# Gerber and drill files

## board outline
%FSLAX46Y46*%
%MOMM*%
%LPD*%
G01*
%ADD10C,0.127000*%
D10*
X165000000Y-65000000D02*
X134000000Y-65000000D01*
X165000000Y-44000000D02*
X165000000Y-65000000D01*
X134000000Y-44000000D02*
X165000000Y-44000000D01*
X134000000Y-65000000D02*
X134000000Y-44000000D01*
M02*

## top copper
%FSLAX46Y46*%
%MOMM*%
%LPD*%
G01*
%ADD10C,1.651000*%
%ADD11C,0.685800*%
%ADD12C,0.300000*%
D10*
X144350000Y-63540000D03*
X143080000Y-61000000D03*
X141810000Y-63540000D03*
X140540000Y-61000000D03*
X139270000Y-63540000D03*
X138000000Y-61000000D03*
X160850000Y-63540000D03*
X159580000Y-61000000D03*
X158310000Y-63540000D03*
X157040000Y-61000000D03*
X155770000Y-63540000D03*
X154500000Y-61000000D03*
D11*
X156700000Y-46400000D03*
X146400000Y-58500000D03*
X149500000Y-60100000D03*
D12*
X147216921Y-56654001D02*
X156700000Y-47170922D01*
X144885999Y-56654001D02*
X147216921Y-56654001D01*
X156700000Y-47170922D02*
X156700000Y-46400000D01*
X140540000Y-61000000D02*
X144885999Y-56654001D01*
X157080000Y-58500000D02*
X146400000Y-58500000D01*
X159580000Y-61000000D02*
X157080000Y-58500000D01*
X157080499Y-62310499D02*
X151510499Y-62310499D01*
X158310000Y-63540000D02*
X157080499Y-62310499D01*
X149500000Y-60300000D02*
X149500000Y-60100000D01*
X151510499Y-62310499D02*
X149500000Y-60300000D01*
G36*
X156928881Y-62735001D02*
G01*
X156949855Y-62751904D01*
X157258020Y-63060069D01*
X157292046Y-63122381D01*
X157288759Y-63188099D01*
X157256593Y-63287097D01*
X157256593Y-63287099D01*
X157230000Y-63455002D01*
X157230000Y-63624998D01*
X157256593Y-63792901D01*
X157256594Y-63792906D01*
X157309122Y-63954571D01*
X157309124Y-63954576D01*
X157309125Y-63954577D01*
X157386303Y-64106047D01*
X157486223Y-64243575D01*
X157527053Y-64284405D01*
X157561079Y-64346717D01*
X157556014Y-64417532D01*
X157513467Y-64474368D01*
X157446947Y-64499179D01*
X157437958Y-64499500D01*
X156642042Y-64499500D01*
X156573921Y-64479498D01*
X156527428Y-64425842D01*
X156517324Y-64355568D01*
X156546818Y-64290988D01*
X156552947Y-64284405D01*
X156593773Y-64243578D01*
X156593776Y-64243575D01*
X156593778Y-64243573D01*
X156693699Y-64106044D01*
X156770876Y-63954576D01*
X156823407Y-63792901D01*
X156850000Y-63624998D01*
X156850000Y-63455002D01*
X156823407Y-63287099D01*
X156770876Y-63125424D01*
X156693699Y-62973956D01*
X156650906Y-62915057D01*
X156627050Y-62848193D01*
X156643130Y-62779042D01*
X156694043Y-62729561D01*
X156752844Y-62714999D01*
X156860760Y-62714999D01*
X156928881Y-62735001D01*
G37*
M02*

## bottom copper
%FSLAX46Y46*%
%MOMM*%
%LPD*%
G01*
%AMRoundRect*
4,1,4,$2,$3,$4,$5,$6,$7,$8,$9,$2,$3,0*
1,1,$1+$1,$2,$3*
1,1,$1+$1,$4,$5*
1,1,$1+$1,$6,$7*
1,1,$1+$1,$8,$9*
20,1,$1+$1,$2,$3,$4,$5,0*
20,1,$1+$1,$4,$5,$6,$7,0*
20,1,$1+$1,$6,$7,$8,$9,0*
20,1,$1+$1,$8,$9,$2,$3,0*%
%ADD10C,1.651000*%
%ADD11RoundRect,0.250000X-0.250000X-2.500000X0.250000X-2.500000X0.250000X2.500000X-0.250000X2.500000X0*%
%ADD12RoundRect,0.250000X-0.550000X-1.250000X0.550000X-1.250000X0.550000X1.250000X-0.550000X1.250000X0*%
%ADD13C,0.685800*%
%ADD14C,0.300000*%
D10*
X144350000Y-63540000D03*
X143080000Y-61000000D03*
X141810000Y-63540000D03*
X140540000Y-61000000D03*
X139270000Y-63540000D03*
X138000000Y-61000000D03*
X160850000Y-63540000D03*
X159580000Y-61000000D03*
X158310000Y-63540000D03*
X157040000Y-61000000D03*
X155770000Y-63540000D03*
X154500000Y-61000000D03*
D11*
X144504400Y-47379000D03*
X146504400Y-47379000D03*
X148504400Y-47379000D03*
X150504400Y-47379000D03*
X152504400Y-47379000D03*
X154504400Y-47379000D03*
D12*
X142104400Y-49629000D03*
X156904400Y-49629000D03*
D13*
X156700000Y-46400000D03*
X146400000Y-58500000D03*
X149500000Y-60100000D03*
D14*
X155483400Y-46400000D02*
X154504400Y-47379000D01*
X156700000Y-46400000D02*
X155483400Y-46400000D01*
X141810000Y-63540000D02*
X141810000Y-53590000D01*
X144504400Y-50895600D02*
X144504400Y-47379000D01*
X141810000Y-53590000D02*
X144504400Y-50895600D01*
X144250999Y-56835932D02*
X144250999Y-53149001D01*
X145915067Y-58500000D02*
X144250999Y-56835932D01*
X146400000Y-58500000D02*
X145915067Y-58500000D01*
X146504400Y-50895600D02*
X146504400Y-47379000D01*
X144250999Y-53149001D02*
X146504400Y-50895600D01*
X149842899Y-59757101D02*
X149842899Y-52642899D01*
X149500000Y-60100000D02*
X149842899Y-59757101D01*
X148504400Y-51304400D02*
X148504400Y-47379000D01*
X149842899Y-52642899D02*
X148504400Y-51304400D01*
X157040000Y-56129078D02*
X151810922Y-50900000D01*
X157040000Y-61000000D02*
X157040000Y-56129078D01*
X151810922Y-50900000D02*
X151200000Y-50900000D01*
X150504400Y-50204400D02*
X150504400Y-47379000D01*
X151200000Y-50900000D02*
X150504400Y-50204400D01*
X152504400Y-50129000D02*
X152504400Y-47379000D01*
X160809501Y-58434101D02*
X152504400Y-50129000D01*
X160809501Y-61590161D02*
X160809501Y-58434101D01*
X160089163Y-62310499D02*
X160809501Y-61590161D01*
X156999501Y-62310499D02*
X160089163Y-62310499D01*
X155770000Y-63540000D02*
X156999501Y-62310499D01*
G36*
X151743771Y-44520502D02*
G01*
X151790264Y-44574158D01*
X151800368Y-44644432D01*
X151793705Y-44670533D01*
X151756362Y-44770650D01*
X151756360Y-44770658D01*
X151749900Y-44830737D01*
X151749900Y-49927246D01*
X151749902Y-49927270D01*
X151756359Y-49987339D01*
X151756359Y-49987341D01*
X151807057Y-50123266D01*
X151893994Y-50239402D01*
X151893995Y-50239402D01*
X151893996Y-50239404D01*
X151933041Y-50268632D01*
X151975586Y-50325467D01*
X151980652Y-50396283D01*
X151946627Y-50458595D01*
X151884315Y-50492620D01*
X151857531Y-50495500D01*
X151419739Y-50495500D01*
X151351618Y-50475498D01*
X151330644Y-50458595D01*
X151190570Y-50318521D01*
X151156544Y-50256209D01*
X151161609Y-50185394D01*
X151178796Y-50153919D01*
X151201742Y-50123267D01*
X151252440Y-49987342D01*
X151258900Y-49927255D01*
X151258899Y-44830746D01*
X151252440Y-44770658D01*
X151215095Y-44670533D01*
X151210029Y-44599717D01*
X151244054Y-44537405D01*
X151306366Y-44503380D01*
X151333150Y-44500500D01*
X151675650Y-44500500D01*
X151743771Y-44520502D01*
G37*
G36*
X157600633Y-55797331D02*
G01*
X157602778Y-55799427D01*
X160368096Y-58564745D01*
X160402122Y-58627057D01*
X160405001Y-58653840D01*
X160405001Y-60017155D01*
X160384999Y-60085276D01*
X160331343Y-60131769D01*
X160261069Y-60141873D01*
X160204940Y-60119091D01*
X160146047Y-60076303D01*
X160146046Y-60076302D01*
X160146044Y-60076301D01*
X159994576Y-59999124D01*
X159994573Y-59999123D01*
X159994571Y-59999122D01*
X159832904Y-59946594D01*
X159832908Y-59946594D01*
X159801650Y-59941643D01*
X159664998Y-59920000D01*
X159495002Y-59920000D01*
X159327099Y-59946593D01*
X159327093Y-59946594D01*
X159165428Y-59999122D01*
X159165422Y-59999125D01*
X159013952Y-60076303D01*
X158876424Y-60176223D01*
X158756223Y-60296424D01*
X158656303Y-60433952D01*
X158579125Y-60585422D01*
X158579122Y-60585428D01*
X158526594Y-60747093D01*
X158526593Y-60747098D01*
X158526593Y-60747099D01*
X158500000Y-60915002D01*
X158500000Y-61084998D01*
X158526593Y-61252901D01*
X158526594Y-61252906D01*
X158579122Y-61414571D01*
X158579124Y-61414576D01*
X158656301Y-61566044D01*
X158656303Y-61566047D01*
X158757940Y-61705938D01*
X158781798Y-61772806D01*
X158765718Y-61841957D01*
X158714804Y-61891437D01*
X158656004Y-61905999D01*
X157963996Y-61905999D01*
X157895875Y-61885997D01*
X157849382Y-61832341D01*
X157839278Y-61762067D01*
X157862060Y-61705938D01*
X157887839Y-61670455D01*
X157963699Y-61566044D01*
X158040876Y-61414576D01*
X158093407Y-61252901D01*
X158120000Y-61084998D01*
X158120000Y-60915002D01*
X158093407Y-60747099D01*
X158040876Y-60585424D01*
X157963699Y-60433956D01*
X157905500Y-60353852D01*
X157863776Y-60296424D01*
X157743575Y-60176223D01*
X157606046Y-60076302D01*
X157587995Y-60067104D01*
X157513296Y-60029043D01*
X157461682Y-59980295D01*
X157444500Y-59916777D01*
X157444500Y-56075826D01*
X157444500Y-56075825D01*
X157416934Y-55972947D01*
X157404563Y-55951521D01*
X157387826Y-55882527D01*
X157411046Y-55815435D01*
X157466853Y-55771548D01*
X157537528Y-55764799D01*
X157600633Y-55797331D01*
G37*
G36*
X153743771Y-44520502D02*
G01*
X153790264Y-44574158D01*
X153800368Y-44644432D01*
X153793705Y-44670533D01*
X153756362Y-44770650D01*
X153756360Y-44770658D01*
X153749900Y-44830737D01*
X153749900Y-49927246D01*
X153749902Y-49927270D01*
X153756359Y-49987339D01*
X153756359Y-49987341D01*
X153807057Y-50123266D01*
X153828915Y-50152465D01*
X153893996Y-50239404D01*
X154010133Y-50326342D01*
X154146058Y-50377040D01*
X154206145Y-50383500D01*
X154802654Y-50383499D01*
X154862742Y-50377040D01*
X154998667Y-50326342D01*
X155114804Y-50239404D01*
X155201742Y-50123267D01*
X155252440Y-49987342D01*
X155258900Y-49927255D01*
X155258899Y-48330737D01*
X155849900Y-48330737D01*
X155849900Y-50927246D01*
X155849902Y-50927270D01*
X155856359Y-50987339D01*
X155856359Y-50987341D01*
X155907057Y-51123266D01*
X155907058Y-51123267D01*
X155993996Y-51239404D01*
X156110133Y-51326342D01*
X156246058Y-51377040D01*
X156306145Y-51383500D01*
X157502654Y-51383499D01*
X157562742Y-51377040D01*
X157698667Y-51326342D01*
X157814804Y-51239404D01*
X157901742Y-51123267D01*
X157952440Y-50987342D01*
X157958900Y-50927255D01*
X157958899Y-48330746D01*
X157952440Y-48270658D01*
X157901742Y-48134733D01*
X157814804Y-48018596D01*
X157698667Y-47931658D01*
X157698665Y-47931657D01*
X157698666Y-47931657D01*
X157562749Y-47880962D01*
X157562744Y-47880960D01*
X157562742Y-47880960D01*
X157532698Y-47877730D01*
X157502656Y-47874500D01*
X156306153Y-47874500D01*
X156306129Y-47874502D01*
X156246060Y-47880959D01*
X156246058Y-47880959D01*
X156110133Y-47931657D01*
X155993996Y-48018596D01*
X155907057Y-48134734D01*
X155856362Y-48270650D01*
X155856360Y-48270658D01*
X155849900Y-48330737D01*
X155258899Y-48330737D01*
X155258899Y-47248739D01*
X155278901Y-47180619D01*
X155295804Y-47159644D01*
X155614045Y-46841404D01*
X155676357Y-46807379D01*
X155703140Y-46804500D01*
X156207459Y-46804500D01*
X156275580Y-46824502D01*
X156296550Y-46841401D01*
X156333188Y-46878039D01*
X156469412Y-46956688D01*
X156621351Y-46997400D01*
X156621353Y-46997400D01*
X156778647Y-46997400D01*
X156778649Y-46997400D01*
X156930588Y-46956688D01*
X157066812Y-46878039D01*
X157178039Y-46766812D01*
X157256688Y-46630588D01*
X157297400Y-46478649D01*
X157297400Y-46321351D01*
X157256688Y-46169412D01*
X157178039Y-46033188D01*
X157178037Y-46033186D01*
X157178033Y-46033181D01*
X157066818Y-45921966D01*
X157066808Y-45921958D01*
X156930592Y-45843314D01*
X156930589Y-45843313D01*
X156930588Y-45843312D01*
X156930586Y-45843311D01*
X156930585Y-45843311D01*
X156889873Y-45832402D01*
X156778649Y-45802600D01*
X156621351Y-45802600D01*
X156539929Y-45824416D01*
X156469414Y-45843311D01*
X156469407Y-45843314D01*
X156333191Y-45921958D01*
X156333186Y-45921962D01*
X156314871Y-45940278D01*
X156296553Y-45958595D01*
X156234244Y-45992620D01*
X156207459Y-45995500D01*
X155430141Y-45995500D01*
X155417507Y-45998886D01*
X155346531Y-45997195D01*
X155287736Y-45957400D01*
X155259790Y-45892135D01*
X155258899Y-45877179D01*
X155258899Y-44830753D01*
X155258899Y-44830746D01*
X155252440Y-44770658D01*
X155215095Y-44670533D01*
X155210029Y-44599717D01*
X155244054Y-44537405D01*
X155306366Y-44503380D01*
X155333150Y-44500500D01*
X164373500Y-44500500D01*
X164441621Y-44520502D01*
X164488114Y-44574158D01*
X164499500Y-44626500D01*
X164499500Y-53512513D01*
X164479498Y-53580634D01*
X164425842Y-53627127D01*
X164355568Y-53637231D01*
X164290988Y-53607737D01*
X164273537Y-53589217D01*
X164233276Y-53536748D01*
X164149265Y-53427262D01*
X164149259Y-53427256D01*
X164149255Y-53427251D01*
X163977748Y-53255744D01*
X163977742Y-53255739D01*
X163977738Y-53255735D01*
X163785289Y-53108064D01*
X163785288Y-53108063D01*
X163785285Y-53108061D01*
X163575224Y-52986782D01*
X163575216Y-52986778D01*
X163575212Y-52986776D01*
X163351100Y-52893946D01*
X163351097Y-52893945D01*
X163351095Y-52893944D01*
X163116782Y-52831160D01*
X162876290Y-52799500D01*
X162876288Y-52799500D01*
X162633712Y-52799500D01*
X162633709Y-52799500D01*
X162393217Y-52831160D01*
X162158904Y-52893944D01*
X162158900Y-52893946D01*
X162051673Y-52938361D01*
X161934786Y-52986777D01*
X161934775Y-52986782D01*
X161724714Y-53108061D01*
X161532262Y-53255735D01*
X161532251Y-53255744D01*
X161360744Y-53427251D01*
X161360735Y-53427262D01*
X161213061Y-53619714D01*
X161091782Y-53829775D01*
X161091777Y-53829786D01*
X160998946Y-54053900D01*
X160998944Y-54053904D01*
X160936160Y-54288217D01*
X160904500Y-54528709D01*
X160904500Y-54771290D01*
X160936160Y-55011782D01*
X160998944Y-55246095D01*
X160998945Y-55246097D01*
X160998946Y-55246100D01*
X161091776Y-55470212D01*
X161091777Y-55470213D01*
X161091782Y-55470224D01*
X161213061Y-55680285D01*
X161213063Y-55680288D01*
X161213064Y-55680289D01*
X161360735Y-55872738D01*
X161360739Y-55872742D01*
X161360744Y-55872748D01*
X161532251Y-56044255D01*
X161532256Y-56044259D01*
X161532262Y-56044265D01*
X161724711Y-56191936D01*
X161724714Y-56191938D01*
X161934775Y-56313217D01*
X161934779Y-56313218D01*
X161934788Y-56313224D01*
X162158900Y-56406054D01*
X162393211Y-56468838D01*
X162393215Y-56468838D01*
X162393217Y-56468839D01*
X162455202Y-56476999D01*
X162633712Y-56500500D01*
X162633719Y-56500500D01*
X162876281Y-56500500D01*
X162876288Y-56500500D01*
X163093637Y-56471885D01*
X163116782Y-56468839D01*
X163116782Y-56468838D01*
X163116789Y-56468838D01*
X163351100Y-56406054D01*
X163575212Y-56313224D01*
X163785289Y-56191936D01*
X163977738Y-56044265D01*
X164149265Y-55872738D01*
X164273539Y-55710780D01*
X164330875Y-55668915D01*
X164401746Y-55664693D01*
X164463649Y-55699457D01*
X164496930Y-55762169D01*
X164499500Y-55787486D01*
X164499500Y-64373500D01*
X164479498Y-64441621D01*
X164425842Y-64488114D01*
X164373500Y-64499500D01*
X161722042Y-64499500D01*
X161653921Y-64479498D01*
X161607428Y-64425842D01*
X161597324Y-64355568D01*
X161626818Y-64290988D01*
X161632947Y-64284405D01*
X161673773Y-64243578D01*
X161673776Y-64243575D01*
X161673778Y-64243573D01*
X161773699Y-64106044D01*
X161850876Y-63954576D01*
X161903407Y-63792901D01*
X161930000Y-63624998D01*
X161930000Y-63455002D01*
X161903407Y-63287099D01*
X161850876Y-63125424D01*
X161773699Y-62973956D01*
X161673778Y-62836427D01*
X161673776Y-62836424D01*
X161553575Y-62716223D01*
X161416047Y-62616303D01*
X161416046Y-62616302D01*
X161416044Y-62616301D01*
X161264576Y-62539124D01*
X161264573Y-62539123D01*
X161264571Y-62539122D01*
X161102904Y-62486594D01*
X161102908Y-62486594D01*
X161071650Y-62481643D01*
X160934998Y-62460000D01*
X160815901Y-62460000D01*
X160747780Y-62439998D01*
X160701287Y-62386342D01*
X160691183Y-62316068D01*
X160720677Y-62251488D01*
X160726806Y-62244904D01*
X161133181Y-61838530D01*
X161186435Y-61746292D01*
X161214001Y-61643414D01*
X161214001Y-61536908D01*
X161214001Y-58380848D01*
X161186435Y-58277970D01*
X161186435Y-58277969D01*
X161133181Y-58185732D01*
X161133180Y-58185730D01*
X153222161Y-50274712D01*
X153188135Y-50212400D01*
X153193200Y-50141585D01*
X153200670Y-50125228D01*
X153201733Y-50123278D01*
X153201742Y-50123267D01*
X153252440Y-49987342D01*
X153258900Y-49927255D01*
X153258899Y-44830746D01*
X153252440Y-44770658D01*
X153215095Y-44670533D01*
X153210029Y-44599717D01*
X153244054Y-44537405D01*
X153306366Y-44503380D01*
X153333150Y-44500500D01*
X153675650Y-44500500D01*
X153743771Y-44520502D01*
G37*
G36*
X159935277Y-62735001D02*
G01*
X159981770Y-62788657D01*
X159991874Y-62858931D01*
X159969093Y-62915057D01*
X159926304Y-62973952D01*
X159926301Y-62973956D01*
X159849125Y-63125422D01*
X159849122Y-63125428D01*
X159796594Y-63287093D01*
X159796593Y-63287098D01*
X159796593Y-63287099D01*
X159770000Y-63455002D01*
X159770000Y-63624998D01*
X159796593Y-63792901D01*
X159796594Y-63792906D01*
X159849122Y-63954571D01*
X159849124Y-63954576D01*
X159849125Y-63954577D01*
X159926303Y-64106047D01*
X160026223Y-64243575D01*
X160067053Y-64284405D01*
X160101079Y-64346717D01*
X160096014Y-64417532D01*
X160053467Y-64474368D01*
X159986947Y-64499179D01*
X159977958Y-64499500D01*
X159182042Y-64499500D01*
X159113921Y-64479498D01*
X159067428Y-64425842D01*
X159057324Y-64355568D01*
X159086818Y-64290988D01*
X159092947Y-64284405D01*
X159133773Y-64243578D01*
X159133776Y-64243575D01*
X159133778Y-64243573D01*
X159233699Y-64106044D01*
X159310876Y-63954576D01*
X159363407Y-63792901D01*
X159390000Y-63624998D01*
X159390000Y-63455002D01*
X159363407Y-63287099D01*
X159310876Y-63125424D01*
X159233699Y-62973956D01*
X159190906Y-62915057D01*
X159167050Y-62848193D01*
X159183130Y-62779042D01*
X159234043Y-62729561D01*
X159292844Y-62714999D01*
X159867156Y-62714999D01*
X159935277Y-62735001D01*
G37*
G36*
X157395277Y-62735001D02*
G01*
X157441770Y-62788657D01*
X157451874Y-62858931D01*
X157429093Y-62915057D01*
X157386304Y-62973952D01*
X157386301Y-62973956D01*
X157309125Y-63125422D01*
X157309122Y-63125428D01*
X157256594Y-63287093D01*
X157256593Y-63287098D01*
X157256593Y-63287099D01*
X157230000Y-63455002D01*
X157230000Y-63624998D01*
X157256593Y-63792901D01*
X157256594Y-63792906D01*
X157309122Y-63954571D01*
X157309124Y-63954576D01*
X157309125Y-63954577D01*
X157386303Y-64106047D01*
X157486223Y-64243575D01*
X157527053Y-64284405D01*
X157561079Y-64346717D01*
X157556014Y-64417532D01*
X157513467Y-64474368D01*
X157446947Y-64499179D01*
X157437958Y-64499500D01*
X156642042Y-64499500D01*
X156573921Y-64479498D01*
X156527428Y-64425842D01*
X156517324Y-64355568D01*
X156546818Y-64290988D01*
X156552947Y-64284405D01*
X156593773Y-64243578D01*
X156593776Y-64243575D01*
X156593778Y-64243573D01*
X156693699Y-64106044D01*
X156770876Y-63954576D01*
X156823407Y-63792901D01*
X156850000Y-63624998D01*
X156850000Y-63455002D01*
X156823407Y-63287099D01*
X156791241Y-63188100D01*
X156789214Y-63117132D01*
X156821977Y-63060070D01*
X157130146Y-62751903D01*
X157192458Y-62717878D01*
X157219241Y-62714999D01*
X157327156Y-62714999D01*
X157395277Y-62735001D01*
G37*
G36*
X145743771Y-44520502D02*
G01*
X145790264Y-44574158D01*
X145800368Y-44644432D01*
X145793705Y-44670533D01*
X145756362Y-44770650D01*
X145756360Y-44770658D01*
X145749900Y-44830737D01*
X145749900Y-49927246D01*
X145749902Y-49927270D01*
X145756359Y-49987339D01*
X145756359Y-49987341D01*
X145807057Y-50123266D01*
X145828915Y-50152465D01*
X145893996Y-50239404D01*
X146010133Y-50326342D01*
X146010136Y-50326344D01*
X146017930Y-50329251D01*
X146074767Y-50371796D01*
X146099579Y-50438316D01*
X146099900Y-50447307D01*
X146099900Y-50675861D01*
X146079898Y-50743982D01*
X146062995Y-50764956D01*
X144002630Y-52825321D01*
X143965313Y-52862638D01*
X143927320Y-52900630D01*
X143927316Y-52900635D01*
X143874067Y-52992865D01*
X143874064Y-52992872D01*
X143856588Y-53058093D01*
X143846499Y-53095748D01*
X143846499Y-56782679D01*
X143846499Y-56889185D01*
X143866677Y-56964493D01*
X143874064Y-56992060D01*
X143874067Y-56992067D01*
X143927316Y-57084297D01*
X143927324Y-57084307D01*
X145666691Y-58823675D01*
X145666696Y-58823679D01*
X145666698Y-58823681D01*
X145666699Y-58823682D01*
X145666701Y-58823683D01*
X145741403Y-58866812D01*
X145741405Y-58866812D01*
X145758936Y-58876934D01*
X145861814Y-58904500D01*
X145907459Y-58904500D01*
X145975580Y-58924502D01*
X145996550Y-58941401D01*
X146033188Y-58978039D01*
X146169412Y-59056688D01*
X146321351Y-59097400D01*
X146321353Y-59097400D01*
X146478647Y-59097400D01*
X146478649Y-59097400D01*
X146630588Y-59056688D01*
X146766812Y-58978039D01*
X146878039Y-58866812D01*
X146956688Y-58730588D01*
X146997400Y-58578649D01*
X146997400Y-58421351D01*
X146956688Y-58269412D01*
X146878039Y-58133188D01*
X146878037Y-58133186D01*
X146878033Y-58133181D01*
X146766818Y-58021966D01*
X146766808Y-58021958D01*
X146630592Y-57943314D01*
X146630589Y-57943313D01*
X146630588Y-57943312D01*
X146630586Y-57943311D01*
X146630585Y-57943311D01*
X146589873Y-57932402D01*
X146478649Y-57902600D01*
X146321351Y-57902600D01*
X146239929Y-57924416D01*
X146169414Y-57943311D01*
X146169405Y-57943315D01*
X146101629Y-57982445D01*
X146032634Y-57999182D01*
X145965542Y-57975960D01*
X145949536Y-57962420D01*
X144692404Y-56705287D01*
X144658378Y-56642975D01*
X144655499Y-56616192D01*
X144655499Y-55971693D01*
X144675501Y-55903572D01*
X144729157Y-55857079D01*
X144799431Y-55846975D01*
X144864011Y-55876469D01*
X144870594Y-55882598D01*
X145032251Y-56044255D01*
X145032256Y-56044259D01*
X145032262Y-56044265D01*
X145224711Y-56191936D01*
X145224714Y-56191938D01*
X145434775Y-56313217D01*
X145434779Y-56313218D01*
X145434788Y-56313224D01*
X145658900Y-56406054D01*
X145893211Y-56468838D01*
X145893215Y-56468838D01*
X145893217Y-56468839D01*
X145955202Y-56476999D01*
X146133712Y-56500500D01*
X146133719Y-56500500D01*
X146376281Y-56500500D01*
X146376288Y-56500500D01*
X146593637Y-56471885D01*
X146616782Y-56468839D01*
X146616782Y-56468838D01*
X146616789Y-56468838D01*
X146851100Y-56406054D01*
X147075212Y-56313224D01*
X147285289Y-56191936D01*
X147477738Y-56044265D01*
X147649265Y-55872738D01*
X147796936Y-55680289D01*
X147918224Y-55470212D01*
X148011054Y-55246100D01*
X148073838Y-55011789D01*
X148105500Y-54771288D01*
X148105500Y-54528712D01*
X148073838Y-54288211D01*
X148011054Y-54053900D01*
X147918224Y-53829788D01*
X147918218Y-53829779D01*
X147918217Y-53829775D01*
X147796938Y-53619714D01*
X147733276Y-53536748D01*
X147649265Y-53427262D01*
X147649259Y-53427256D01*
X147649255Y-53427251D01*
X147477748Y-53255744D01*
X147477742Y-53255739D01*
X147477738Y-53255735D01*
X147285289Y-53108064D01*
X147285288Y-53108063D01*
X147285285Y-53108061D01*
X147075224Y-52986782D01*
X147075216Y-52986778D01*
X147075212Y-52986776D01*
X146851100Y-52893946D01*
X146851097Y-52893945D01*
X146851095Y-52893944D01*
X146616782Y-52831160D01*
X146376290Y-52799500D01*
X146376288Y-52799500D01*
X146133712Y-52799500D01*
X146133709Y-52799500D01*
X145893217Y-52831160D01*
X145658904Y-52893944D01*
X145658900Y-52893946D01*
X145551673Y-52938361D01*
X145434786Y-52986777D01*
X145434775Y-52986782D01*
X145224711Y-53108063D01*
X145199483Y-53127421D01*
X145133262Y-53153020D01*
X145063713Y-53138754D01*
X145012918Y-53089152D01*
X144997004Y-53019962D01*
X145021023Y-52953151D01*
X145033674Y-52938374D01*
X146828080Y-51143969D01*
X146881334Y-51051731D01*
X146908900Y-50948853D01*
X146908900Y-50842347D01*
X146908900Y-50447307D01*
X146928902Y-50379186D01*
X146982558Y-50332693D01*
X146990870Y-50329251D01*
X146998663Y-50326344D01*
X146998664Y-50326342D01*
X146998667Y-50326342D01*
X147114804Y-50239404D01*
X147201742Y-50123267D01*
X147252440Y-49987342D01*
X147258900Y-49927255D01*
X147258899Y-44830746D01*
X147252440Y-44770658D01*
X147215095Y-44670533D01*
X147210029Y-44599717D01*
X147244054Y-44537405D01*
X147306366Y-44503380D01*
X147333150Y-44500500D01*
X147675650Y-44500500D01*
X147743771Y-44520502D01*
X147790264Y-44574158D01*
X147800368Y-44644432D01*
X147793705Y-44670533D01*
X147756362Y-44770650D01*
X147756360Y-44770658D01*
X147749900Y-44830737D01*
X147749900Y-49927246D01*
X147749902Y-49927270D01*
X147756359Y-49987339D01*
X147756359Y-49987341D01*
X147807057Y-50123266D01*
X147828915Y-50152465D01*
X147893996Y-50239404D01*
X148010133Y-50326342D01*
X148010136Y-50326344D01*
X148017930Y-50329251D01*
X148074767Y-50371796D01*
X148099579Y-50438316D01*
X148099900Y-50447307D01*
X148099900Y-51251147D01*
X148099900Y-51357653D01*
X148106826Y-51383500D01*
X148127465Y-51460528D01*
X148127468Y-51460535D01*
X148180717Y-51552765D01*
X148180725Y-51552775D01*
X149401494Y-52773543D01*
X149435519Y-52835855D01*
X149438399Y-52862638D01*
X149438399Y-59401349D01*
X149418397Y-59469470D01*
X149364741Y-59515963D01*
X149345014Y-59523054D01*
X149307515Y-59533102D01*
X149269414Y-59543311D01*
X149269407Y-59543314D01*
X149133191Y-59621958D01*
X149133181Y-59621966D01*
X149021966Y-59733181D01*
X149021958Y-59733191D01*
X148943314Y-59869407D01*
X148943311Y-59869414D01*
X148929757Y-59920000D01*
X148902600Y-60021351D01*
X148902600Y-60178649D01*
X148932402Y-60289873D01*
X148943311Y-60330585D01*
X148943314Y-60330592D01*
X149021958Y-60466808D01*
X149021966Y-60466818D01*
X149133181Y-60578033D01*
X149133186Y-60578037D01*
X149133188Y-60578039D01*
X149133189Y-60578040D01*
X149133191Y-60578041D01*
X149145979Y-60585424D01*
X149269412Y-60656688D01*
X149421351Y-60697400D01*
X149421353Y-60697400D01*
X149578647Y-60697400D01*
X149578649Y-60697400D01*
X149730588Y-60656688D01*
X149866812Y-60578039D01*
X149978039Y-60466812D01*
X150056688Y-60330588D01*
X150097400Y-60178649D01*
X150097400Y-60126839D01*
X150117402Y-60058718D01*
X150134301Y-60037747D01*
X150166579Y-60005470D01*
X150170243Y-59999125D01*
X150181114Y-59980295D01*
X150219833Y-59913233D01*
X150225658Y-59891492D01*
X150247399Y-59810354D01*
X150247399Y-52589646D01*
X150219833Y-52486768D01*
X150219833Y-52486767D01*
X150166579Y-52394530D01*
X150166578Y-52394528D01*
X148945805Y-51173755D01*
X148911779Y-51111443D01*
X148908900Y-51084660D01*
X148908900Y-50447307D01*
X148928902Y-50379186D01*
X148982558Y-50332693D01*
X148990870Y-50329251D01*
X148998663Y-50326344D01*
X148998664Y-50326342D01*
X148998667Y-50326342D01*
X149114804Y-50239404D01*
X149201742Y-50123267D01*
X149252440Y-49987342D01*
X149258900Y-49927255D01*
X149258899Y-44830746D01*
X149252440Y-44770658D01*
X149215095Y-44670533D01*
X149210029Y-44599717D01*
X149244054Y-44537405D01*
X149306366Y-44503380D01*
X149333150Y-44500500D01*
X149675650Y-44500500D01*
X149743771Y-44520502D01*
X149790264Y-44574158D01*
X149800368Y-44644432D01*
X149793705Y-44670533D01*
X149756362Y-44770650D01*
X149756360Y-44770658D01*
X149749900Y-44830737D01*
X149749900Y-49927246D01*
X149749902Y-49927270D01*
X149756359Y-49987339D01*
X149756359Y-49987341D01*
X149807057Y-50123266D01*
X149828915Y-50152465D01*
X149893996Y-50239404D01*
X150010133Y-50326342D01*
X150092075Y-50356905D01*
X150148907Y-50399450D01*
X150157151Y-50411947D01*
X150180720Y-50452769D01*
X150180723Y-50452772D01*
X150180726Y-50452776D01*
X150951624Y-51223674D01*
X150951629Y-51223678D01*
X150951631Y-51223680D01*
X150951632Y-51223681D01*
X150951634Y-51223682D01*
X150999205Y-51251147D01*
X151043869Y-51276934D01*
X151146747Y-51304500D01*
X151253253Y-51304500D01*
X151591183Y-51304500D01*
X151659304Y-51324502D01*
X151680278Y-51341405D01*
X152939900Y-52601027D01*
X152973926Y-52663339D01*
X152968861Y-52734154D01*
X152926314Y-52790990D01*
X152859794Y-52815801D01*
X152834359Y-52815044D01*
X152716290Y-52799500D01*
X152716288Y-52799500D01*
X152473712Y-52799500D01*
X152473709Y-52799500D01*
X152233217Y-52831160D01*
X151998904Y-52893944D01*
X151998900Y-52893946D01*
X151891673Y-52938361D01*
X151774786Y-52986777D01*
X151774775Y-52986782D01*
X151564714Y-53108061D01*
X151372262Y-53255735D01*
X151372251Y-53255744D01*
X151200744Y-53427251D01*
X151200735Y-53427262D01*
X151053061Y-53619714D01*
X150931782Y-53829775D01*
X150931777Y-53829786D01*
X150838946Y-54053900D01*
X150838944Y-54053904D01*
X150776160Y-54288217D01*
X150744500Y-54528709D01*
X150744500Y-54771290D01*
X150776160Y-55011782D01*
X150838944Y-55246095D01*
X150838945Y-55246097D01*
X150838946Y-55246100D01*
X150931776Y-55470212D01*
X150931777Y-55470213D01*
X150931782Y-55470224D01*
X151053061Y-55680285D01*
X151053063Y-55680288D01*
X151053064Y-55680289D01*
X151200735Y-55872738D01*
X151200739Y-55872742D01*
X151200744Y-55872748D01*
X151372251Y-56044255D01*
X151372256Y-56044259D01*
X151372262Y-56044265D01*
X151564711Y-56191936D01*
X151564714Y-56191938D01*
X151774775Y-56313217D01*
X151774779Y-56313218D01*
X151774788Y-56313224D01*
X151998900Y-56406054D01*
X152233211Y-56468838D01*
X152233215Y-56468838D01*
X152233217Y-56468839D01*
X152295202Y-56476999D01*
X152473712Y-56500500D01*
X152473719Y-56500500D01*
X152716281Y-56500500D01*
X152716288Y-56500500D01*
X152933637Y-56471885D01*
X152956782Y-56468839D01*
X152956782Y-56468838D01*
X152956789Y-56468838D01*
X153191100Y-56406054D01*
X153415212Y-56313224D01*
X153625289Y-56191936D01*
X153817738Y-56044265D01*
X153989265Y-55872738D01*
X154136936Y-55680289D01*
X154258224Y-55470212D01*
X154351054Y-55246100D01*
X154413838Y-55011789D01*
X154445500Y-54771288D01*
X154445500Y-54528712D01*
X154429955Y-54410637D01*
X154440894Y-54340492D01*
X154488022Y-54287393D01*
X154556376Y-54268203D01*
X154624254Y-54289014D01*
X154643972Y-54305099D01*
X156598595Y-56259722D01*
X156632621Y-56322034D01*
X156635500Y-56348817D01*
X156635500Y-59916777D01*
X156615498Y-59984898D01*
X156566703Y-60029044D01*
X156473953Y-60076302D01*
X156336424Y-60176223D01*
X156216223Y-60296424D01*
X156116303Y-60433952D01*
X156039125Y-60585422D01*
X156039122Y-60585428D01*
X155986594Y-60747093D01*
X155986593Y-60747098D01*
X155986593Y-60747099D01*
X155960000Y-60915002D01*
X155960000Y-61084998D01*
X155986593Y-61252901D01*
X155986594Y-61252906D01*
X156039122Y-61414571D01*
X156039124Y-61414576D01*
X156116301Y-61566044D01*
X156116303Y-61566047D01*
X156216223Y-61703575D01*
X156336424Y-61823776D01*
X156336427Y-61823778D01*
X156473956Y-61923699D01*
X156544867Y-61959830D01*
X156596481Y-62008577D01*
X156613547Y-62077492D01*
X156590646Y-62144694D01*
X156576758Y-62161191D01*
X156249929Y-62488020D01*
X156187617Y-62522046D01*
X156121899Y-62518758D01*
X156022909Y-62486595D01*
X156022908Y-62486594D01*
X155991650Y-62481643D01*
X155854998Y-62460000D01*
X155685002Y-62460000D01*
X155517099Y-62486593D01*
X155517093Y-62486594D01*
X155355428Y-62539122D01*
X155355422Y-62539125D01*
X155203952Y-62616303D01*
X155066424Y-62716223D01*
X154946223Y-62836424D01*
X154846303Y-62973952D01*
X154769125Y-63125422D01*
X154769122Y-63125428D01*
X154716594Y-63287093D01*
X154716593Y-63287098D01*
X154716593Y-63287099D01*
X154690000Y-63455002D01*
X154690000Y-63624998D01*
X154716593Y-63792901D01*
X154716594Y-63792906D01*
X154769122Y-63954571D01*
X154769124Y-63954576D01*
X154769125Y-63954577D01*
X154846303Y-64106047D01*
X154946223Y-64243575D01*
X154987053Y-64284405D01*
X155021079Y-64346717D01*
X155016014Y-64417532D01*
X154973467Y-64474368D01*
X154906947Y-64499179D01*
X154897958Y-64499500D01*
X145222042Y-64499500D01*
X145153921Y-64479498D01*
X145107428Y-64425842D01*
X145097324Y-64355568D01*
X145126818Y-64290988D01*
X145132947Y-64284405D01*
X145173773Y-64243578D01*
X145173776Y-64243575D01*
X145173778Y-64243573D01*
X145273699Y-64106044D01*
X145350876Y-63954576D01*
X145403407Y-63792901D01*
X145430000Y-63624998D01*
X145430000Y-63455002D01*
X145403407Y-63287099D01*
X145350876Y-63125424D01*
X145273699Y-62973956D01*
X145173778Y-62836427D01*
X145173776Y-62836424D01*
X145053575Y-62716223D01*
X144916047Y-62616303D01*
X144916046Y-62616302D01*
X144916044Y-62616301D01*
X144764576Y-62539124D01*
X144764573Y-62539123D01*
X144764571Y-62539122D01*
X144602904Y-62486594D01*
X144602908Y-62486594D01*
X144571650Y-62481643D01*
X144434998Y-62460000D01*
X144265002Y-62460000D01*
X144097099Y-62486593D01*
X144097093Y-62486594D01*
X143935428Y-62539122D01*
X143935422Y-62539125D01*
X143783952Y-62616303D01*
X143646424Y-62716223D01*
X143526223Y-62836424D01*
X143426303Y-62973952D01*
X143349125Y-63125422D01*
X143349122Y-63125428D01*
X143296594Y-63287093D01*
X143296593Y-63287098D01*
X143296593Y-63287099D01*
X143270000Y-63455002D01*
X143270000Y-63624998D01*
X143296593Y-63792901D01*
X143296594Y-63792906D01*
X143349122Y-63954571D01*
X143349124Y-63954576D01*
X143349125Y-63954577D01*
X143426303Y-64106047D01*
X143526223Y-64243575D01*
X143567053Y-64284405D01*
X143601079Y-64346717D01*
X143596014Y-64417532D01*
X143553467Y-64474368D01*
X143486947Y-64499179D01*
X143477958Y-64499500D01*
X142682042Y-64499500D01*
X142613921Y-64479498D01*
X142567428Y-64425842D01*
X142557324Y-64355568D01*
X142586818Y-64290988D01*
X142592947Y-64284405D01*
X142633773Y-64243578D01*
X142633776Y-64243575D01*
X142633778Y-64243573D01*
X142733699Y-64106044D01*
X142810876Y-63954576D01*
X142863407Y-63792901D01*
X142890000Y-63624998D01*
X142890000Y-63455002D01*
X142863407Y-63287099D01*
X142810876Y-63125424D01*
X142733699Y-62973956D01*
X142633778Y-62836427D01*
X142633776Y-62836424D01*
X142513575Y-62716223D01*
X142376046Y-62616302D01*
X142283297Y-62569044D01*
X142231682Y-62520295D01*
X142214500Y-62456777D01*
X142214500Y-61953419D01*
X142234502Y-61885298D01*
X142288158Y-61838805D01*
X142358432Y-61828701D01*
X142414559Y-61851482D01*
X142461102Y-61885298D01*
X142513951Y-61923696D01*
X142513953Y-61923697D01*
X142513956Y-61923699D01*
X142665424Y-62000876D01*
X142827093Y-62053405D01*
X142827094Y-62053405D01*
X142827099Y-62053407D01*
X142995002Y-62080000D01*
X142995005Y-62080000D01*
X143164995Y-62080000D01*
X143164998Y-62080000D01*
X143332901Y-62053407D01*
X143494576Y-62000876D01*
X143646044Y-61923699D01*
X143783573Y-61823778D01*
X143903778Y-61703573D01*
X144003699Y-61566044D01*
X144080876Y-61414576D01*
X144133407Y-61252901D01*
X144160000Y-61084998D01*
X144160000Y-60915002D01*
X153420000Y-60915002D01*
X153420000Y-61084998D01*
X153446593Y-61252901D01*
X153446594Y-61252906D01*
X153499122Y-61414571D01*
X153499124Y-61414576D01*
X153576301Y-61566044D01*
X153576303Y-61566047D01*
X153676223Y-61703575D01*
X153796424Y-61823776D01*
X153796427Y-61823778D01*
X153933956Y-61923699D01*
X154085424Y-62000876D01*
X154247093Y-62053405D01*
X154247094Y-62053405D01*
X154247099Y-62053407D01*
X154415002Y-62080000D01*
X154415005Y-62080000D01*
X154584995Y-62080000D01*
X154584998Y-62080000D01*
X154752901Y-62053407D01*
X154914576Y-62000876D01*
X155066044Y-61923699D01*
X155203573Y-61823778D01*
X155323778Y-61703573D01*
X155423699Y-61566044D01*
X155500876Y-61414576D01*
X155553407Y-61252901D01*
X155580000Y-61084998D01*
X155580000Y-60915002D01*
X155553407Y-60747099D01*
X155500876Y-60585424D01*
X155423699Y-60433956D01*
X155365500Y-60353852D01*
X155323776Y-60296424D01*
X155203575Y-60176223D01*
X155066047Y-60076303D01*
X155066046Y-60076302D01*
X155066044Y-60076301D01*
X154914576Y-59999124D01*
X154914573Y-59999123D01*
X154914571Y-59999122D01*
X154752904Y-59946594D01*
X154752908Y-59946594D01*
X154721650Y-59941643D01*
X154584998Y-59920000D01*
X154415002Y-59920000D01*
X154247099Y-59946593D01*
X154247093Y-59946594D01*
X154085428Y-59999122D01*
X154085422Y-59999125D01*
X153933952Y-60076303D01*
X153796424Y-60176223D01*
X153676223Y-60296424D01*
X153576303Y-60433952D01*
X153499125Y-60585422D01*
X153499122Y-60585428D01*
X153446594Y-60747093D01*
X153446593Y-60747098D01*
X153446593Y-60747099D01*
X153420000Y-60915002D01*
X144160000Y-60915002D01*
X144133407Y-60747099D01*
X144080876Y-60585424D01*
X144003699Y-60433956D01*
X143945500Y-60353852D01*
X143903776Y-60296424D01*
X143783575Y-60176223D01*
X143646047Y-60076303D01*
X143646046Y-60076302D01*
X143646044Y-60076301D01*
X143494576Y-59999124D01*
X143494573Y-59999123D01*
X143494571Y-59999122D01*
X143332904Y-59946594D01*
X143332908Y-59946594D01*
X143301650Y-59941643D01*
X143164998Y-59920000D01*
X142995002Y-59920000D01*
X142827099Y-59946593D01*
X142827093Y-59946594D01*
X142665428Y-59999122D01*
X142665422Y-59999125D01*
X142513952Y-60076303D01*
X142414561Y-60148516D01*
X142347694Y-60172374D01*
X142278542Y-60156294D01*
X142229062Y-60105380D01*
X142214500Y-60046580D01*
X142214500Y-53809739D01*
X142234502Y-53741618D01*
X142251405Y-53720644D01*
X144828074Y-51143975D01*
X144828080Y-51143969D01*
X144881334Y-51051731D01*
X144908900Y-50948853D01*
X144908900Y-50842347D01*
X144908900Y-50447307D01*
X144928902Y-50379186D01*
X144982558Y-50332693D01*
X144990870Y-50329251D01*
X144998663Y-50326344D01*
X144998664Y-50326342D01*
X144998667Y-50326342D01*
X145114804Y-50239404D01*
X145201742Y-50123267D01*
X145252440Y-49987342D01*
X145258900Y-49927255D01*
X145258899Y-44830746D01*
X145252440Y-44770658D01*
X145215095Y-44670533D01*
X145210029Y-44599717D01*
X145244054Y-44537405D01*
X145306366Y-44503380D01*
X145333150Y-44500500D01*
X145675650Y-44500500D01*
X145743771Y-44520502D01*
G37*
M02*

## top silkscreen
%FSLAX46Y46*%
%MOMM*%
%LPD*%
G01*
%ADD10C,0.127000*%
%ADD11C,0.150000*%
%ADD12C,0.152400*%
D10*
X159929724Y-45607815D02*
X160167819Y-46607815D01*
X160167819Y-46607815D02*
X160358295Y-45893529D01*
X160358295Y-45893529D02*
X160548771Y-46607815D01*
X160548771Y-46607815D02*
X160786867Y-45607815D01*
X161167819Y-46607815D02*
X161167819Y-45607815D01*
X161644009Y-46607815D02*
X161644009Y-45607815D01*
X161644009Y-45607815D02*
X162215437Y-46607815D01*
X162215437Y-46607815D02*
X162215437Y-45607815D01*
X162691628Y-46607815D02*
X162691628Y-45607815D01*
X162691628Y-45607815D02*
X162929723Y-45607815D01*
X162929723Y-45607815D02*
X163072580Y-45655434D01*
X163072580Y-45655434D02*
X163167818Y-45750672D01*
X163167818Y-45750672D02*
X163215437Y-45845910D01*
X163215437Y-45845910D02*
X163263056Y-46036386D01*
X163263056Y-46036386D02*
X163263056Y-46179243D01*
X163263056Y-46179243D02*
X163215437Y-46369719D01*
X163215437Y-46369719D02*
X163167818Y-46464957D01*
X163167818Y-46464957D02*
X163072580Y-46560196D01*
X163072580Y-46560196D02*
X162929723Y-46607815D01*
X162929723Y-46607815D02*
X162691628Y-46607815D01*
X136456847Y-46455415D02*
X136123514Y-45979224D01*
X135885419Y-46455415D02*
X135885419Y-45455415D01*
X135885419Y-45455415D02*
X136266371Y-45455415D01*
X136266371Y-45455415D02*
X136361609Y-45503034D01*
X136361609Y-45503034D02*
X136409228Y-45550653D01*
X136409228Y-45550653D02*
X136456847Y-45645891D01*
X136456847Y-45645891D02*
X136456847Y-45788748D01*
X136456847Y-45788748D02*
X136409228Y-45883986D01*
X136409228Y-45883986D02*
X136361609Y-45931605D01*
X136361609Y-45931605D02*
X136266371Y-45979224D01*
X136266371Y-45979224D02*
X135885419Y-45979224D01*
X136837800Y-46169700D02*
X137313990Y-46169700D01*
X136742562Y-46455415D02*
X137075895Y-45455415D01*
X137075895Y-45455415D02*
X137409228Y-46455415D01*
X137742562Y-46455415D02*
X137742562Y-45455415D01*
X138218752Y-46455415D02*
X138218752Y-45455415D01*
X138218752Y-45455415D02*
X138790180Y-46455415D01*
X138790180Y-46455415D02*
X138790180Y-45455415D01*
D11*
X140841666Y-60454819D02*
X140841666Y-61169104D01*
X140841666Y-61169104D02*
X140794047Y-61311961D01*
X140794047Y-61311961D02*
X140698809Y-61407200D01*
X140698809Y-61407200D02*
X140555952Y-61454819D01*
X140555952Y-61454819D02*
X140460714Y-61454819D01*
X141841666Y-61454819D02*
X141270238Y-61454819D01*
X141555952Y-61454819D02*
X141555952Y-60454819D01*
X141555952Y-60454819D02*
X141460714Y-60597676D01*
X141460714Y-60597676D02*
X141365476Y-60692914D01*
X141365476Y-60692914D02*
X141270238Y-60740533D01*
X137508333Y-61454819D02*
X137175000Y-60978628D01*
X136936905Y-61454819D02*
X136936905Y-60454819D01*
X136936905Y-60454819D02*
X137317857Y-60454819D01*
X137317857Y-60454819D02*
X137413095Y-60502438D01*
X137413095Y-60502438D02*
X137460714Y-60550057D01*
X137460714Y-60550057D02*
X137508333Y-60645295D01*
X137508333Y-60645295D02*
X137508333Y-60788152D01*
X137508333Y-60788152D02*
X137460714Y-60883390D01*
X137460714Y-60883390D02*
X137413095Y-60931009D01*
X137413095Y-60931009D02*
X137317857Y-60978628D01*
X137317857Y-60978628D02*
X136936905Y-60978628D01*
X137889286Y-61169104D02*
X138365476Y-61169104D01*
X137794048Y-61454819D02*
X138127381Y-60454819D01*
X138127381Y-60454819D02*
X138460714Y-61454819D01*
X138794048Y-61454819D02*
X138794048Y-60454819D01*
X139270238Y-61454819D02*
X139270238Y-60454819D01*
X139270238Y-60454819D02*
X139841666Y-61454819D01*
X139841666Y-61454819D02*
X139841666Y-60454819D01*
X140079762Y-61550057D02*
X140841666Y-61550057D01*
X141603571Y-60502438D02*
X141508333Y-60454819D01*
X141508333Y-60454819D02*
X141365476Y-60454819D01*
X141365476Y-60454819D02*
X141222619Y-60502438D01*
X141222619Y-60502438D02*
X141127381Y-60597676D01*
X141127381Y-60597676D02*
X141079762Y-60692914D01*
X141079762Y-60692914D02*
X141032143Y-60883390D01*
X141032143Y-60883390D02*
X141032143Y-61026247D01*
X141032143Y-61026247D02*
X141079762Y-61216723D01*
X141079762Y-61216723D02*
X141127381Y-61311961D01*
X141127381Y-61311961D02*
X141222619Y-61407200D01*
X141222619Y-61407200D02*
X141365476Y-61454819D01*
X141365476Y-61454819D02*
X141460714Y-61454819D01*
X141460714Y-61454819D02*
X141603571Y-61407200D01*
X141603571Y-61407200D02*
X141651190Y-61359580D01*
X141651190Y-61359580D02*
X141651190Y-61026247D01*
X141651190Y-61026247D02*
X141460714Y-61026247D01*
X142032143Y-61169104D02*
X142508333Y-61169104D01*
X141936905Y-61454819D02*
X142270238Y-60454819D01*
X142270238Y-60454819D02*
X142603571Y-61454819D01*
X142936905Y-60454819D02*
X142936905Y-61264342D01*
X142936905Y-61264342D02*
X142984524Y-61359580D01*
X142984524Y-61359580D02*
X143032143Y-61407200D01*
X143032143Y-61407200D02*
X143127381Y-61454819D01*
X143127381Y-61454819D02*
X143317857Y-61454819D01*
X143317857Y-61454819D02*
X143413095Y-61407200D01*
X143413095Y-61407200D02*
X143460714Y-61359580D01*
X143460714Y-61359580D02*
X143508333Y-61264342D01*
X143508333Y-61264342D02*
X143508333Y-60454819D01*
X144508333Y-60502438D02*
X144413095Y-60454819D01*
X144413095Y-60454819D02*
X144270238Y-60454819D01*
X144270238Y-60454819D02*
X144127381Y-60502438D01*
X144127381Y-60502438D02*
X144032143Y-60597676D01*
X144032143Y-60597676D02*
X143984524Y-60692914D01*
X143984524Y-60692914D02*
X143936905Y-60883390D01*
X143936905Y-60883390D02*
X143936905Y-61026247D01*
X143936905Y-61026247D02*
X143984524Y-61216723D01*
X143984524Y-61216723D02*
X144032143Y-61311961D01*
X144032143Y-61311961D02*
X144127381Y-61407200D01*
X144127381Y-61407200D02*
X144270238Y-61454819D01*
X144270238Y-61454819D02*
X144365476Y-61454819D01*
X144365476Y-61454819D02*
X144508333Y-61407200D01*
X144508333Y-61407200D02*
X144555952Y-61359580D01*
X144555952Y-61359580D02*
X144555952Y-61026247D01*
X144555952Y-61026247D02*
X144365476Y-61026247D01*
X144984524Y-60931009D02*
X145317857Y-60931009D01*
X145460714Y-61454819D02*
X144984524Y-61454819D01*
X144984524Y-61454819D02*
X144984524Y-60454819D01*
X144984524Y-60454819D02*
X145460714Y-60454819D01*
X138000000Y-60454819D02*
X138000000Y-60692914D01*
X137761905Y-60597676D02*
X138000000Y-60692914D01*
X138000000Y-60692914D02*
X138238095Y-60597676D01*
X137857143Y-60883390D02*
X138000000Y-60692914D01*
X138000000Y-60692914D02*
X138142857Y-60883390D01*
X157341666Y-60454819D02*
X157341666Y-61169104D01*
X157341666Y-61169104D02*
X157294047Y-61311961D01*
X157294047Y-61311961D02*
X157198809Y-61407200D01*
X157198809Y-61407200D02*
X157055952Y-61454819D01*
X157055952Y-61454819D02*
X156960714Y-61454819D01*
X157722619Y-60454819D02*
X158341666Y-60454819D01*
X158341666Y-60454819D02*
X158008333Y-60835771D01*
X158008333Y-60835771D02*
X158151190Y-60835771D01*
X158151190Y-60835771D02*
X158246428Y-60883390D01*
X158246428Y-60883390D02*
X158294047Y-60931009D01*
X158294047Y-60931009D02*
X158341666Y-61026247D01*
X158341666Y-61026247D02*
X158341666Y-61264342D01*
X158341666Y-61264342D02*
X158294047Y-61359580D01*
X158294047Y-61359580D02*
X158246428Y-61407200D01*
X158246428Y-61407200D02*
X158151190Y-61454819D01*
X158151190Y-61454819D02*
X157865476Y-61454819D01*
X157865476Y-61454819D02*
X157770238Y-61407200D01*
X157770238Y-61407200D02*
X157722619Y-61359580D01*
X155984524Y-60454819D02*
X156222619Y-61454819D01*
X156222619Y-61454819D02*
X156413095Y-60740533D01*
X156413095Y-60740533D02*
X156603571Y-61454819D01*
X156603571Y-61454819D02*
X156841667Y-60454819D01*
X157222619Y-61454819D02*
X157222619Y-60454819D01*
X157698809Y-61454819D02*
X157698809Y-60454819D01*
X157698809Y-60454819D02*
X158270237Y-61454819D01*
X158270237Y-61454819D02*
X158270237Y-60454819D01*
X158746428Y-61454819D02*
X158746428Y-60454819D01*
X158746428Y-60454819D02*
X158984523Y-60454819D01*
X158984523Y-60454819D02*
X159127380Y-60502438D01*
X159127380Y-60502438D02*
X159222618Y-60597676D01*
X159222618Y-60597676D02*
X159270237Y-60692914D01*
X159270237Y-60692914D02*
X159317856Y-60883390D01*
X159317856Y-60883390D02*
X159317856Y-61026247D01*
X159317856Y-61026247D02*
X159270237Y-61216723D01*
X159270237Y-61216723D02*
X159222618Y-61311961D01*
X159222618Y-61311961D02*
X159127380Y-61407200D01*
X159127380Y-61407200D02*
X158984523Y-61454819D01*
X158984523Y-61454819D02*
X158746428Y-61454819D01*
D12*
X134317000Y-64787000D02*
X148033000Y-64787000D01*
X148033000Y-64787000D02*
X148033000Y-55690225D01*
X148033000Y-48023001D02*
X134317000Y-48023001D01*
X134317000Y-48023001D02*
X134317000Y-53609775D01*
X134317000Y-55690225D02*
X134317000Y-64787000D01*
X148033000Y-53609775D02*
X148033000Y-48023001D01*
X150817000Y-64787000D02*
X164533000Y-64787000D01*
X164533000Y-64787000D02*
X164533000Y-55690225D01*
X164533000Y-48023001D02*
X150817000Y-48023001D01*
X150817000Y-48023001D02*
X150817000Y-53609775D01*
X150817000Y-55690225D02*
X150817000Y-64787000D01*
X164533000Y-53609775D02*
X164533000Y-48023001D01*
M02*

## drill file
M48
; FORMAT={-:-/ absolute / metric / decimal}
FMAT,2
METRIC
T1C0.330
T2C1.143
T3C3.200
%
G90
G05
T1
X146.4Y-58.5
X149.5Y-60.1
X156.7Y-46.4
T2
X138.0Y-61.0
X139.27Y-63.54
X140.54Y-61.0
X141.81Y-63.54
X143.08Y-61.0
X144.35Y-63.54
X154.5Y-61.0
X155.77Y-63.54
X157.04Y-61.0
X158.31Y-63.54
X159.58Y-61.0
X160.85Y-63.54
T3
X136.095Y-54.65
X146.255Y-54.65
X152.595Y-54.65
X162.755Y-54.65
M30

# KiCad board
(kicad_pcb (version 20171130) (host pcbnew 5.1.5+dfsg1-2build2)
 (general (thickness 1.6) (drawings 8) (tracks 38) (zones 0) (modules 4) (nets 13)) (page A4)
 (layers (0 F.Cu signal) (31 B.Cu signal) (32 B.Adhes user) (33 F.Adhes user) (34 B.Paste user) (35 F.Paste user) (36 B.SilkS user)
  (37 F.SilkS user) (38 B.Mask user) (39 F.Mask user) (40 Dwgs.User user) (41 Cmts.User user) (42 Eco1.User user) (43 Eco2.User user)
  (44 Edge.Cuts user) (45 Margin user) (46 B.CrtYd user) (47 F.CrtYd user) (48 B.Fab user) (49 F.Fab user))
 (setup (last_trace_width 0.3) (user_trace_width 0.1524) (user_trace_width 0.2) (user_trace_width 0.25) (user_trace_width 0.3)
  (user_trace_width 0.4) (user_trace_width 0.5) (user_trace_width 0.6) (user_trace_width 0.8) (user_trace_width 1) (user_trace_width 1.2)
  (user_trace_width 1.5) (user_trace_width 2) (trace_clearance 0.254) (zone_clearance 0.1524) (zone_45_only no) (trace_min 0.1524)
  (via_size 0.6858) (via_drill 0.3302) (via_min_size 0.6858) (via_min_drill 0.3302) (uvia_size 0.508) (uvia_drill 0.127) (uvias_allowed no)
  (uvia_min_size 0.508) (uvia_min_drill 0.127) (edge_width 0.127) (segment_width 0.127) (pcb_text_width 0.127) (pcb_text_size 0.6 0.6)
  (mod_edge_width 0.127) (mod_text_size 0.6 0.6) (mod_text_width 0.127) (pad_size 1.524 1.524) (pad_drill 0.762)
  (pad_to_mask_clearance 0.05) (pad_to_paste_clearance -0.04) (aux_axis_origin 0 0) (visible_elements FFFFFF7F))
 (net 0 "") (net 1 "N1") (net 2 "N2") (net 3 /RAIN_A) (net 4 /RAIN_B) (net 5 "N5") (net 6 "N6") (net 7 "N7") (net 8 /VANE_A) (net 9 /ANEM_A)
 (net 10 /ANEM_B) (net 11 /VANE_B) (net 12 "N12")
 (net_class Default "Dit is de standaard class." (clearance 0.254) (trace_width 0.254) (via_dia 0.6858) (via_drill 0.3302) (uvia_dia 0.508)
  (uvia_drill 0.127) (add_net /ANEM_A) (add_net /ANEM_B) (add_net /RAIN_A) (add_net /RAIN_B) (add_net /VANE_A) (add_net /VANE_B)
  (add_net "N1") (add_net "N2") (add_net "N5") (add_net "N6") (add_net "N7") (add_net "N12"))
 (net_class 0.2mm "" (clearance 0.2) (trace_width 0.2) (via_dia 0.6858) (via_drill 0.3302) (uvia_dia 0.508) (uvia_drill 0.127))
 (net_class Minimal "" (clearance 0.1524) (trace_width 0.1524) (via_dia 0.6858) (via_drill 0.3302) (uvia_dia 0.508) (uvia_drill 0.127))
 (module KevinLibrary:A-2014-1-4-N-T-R (layer F.Cu) (at 138 61)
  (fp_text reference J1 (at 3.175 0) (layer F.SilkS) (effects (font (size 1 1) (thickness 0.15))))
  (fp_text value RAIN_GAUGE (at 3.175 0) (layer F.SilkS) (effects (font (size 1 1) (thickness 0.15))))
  (fp_line (start -3.683 3.787) (end 10.033 3.787) (layer F.SilkS) (width 0.1524))
  (fp_line (start 10.033 3.787) (end 10.033 -5.309775) (layer F.SilkS) (width 0.1524))
  (fp_line (start 10.033 -12.976999) (end -3.683 -12.976999) (layer F.SilkS) (width 0.1524))
  (fp_line (start -3.683 -12.976999) (end -3.683 -7.390225) (layer F.SilkS) (width 0.1524))
  (fp_line (start -3.683 -5.309775) (end -3.683 3.787) (layer F.SilkS) (width 0.1524))
  (fp_line (start 10.033 -7.390225) (end 10.033 -12.976999) (layer F.SilkS) (width 0.1524))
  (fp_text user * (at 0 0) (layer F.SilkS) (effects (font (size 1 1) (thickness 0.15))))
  (pad 1 thru_hole circle (at 6.35 2.54) (size 1.651 1.651) (drill 1.143) (layers *.Cu *.Mask) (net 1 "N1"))
  (pad 2 thru_hole circle (at 5.08 0) (size 1.651 1.651) (drill 1.143) (layers *.Cu *.Mask) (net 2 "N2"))
  (pad 3 thru_hole circle (at 3.81 2.54) (size 1.651 1.651) (drill 1.143) (layers *.Cu *.Mask) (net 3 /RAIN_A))
  (pad 4 thru_hole circle (at 2.54 0) (size 1.651 1.651) (drill 1.143) (layers *.Cu *.Mask) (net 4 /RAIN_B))
  (pad 5 thru_hole circle (at 1.27 2.54) (size 1.651 1.651) (drill 1.143) (layers *.Cu *.Mask) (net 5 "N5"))
  (pad 6 thru_hole circle (at 0 0) (size 1.651 1.651) (drill 1.143) (layers *.Cu *.Mask) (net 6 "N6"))
  (pad "" np_thru_hole circle (at -1.905 -6.35 90) (size 3.2 3.2) (drill 3.2) (layers *.Cu))
  (pad "" np_thru_hole circle (at 8.255 -6.35 90) (size 3.2 3.2) (drill 3.2) (layers *.Cu)))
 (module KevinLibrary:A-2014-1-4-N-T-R (layer F.Cu) (at 154.5 61)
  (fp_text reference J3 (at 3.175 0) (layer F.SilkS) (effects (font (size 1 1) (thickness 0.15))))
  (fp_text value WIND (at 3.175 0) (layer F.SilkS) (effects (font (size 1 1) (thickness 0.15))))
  (fp_line (start -3.683 3.787) (end 10.033 3.787) (layer F.SilkS) (width 0.1524))
  (fp_line (start 10.033 3.787) (end 10.033 -5.309775) (layer F.SilkS) (width 0.1524))
  (fp_line (start 10.033 -12.976999) (end -3.683 -12.976999) (layer F.SilkS) (width 0.1524))
  (fp_line (start -3.683 -12.976999) (end -3.683 -7.390225) (layer F.SilkS) (width 0.1524))
  (fp_line (start -3.683 -5.309775) (end -3.683 3.787) (layer F.SilkS) (width 0.1524))
  (fp_line (start 10.033 -7.390225) (end 10.033 -12.976999) (layer F.SilkS) (width 0.1524))
  (pad 1 thru_hole circle (at 6.35 2.54) (size 1.651 1.651) (drill 1.143) (layers *.Cu *.Mask) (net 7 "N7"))
  (pad 2 thru_hole circle (at 5.08 0) (size 1.651 1.651) (drill 1.143) (layers *.Cu *.Mask) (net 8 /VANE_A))
  (pad 3 thru_hole circle (at 3.81 2.54) (size 1.651 1.651) (drill 1.143) (layers *.Cu *.Mask) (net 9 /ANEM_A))
  (pad 4 thru_hole circle (at 2.54 0) (size 1.651 1.651) (drill 1.143) (layers *.Cu *.Mask) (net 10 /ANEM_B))
  (pad 5 thru_hole circle (at 1.27 2.54) (size 1.651 1.651) (drill 1.143) (layers *.Cu *.Mask) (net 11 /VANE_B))
  (pad 6 thru_hole circle (at 0 0) (size 1.651 1.651) (drill 1.143) (layers *.Cu *.Mask) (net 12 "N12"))
  (pad "" np_thru_hole circle (at -1.905 -6.35 90) (size 3.2 3.2) (drill 3.2) (layers *.Cu))
  (pad "" np_thru_hole circle (at 8.255 -6.35 90) (size 3.2 3.2) (drill 3.2) (layers *.Cu)))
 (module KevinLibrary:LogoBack (layer F.Cu) (at 161.2646 50.0126)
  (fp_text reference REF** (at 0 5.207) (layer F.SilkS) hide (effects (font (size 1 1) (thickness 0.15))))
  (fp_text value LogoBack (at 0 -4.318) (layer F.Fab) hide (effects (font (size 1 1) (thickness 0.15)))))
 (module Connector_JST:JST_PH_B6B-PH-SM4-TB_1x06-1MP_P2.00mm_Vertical (layer B.Cu) (at 149.5044 47.879)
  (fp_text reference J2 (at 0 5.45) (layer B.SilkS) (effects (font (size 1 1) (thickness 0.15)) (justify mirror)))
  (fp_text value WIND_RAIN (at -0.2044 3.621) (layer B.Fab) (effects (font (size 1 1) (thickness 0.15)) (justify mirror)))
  (pad 1 smd roundrect (at -5 -0.5) (size 1 5.5) (layers B.Cu B.Paste B.Mask) (roundrect_rratio 0.25) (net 3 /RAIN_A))
  (pad 2 smd roundrect (at -3 -0.5) (size 1 5.5) (layers B.Cu B.Paste B.Mask) (roundrect_rratio 0.25) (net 8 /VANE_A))
  (pad 3 smd roundrect (at -1 -0.5) (size 1 5.5) (layers B.Cu B.Paste B.Mask) (roundrect_rratio 0.25) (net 9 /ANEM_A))
  (pad 4 smd roundrect (at 1 -0.5) (size 1 5.5) (layers B.Cu B.Paste B.Mask) (roundrect_rratio 0.25) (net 10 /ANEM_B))
  (pad 5 smd roundrect (at 3 -0.5) (size 1 5.5) (layers B.Cu B.Paste B.Mask) (roundrect_rratio 0.25) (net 11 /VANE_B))
  (pad 6 smd roundrect (at 5 -0.5) (size 1 5.5) (layers B.Cu B.Paste B.Mask) (roundrect_rratio 0.25) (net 4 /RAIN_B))
  (pad MP smd roundrect (at -7.4 1.75) (size 1.6 3) (layers B.Cu B.Paste B.Mask) (roundrect_rratio 0.15625))
  (pad MP smd roundrect (at 7.4 1.75) (size 1.6 3) (layers B.Cu B.Paste B.Mask) (roundrect_rratio 0.15625)))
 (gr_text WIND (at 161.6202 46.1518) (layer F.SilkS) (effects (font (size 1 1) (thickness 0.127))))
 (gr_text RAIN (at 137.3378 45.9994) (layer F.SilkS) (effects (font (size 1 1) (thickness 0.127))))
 (gr_line (start 165 65) (end 134 65) (layer Edge.Cuts) (width 0.127))
 (gr_line (start 165 44) (end 165 65) (layer Edge.Cuts) (width 0.127))
 (gr_line (start 134 44) (end 165 44) (layer Edge.Cuts) (width 0.127))
 (gr_line (start 134 65) (end 134 44) (layer Edge.Cuts) (width 0.127))
 (via (at 156.7 46.4) (size 0.6858) (drill 0.3302) (layers F.Cu B.Cu) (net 4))
 (segment (start 147.216921 56.654001) (end 156.7 47.170922) (width 0.3) (layer F.Cu) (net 4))
 (segment (start 144.885999 56.654001) (end 147.216921 56.654001) (width 0.3) (layer F.Cu) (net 4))
 (segment (start 156.7 47.170922) (end 156.7 46.4) (width 0.3) (layer F.Cu) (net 4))
 (segment (start 140.54 61) (end 144.885999 56.654001) (width 0.3) (layer F.Cu) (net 4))
 (segment (start 155.4834 46.4) (end 154.5044 47.379) (width 0.3) (layer B.Cu) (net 4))
 (segment (start 156.7 46.4) (end 155.4834 46.4) (width 0.3) (layer B.Cu) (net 4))
 (segment (start 141.81 63.54) (end 141.81 53.59) (width 0.3) (layer B.Cu) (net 3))
 (segment (start 144.5044 50.8956) (end 144.5044 47.379) (width 0.3) (layer B.Cu) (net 3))
 (segment (start 141.81 53.59) (end 144.5044 50.8956) (width 0.3) (layer B.Cu) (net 3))
 (segment (start 157.08 58.5) (end 146.4 58.5) (width 0.3) (layer F.Cu) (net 8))
 (via (at 146.4 58.5) (size 0.6858) (drill 0.3302) (layers F.Cu B.Cu) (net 8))
 (segment (start 159.58 61) (end 157.08 58.5) (width 0.3) (layer F.Cu) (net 8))
 (segment (start 144.250999 56.835932) (end 144.250999 53.149001) (width 0.3) (layer B.Cu) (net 8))
 (segment (start 145.915067 58.5) (end 144.250999 56.835932) (width 0.3) (layer B.Cu) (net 8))
 (segment (start 146.4 58.5) (end 145.915067 58.5) (width 0.3) (layer B.Cu) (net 8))
 (segment (start 146.5044 50.8956) (end 146.5044 47.379) (width 0.3) (layer B.Cu) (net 8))
 (segment (start 144.250999 53.149001) (end 146.5044 50.8956) (width 0.3) (layer B.Cu) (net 8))
 (segment (start 157.080499 62.310499) (end 151.510499 62.310499) (width 0.3) (layer F.Cu) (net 9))
 (segment (start 158.31 63.54) (end 157.080499 62.310499) (width 0.3) (layer F.Cu) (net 9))
 (via (at 149.5 60.1) (size 0.6858) (drill 0.3302) (layers F.Cu B.Cu) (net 9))
 (segment (start 149.5 60.3) (end 149.5 60.1) (width 0.3) (layer F.Cu) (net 9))
 (segment (start 151.510499 62.310499) (end 149.5 60.3) (width 0.3) (layer F.Cu) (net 9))
 (segment (start 149.842899 59.757101) (end 149.842899 52.642899) (width 0.3) (layer B.Cu) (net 9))
 (segment (start 149.5 60.1) (end 149.842899 59.757101) (width 0.3) (layer B.Cu) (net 9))
 (segment (start 148.5044 51.3044) (end 148.5044 47.379) (width 0.3) (layer B.Cu) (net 9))
 (segment (start 149.842899 52.642899) (end 148.5044 51.3044) (width 0.3) (layer B.Cu) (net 9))
 (segment (start 157.04 56.129078) (end 151.810922 50.9) (width 0.3) (layer B.Cu) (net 10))
 (segment (start 157.04 61) (end 157.04 56.129078) (width 0.3) (layer B.Cu) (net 10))
 (segment (start 151.810922 50.9) (end 151.2 50.9) (width 0.3) (layer B.Cu) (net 10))
 (segment (start 150.5044 50.2044) (end 150.5044 47.379) (width 0.3) (layer B.Cu) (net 10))
 (segment (start 151.2 50.9) (end 150.5044 50.2044) (width 0.3) (layer B.Cu) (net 10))
 (segment (start 152.5044 50.129) (end 152.5044 47.379) (width 0.3) (layer B.Cu) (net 11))
 (segment (start 160.809501 58.434101) (end 152.5044 50.129) (width 0.3) (layer B.Cu) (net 11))
 (segment (start 160.809501 61.590161) (end 160.809501 58.434101) (width 0.3) (layer B.Cu) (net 11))
 (segment (start 160.089163 62.310499) (end 160.809501 61.590161) (width 0.3) (layer B.Cu) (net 11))
 (segment (start 156.999501 62.310499) (end 160.089163 62.310499) (width 0.3) (layer B.Cu) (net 11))
 (segment (start 155.77 63.54) (end 156.999501 62.310499) (width 0.3) (layer B.Cu) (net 11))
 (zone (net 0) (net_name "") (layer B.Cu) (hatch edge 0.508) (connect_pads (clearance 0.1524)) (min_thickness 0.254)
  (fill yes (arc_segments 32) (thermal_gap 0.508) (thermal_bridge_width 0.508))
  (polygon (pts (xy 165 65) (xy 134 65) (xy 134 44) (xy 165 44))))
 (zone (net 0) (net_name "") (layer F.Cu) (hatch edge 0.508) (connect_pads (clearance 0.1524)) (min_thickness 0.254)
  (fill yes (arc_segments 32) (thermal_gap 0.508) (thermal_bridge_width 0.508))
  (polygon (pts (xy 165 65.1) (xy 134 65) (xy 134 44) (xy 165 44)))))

